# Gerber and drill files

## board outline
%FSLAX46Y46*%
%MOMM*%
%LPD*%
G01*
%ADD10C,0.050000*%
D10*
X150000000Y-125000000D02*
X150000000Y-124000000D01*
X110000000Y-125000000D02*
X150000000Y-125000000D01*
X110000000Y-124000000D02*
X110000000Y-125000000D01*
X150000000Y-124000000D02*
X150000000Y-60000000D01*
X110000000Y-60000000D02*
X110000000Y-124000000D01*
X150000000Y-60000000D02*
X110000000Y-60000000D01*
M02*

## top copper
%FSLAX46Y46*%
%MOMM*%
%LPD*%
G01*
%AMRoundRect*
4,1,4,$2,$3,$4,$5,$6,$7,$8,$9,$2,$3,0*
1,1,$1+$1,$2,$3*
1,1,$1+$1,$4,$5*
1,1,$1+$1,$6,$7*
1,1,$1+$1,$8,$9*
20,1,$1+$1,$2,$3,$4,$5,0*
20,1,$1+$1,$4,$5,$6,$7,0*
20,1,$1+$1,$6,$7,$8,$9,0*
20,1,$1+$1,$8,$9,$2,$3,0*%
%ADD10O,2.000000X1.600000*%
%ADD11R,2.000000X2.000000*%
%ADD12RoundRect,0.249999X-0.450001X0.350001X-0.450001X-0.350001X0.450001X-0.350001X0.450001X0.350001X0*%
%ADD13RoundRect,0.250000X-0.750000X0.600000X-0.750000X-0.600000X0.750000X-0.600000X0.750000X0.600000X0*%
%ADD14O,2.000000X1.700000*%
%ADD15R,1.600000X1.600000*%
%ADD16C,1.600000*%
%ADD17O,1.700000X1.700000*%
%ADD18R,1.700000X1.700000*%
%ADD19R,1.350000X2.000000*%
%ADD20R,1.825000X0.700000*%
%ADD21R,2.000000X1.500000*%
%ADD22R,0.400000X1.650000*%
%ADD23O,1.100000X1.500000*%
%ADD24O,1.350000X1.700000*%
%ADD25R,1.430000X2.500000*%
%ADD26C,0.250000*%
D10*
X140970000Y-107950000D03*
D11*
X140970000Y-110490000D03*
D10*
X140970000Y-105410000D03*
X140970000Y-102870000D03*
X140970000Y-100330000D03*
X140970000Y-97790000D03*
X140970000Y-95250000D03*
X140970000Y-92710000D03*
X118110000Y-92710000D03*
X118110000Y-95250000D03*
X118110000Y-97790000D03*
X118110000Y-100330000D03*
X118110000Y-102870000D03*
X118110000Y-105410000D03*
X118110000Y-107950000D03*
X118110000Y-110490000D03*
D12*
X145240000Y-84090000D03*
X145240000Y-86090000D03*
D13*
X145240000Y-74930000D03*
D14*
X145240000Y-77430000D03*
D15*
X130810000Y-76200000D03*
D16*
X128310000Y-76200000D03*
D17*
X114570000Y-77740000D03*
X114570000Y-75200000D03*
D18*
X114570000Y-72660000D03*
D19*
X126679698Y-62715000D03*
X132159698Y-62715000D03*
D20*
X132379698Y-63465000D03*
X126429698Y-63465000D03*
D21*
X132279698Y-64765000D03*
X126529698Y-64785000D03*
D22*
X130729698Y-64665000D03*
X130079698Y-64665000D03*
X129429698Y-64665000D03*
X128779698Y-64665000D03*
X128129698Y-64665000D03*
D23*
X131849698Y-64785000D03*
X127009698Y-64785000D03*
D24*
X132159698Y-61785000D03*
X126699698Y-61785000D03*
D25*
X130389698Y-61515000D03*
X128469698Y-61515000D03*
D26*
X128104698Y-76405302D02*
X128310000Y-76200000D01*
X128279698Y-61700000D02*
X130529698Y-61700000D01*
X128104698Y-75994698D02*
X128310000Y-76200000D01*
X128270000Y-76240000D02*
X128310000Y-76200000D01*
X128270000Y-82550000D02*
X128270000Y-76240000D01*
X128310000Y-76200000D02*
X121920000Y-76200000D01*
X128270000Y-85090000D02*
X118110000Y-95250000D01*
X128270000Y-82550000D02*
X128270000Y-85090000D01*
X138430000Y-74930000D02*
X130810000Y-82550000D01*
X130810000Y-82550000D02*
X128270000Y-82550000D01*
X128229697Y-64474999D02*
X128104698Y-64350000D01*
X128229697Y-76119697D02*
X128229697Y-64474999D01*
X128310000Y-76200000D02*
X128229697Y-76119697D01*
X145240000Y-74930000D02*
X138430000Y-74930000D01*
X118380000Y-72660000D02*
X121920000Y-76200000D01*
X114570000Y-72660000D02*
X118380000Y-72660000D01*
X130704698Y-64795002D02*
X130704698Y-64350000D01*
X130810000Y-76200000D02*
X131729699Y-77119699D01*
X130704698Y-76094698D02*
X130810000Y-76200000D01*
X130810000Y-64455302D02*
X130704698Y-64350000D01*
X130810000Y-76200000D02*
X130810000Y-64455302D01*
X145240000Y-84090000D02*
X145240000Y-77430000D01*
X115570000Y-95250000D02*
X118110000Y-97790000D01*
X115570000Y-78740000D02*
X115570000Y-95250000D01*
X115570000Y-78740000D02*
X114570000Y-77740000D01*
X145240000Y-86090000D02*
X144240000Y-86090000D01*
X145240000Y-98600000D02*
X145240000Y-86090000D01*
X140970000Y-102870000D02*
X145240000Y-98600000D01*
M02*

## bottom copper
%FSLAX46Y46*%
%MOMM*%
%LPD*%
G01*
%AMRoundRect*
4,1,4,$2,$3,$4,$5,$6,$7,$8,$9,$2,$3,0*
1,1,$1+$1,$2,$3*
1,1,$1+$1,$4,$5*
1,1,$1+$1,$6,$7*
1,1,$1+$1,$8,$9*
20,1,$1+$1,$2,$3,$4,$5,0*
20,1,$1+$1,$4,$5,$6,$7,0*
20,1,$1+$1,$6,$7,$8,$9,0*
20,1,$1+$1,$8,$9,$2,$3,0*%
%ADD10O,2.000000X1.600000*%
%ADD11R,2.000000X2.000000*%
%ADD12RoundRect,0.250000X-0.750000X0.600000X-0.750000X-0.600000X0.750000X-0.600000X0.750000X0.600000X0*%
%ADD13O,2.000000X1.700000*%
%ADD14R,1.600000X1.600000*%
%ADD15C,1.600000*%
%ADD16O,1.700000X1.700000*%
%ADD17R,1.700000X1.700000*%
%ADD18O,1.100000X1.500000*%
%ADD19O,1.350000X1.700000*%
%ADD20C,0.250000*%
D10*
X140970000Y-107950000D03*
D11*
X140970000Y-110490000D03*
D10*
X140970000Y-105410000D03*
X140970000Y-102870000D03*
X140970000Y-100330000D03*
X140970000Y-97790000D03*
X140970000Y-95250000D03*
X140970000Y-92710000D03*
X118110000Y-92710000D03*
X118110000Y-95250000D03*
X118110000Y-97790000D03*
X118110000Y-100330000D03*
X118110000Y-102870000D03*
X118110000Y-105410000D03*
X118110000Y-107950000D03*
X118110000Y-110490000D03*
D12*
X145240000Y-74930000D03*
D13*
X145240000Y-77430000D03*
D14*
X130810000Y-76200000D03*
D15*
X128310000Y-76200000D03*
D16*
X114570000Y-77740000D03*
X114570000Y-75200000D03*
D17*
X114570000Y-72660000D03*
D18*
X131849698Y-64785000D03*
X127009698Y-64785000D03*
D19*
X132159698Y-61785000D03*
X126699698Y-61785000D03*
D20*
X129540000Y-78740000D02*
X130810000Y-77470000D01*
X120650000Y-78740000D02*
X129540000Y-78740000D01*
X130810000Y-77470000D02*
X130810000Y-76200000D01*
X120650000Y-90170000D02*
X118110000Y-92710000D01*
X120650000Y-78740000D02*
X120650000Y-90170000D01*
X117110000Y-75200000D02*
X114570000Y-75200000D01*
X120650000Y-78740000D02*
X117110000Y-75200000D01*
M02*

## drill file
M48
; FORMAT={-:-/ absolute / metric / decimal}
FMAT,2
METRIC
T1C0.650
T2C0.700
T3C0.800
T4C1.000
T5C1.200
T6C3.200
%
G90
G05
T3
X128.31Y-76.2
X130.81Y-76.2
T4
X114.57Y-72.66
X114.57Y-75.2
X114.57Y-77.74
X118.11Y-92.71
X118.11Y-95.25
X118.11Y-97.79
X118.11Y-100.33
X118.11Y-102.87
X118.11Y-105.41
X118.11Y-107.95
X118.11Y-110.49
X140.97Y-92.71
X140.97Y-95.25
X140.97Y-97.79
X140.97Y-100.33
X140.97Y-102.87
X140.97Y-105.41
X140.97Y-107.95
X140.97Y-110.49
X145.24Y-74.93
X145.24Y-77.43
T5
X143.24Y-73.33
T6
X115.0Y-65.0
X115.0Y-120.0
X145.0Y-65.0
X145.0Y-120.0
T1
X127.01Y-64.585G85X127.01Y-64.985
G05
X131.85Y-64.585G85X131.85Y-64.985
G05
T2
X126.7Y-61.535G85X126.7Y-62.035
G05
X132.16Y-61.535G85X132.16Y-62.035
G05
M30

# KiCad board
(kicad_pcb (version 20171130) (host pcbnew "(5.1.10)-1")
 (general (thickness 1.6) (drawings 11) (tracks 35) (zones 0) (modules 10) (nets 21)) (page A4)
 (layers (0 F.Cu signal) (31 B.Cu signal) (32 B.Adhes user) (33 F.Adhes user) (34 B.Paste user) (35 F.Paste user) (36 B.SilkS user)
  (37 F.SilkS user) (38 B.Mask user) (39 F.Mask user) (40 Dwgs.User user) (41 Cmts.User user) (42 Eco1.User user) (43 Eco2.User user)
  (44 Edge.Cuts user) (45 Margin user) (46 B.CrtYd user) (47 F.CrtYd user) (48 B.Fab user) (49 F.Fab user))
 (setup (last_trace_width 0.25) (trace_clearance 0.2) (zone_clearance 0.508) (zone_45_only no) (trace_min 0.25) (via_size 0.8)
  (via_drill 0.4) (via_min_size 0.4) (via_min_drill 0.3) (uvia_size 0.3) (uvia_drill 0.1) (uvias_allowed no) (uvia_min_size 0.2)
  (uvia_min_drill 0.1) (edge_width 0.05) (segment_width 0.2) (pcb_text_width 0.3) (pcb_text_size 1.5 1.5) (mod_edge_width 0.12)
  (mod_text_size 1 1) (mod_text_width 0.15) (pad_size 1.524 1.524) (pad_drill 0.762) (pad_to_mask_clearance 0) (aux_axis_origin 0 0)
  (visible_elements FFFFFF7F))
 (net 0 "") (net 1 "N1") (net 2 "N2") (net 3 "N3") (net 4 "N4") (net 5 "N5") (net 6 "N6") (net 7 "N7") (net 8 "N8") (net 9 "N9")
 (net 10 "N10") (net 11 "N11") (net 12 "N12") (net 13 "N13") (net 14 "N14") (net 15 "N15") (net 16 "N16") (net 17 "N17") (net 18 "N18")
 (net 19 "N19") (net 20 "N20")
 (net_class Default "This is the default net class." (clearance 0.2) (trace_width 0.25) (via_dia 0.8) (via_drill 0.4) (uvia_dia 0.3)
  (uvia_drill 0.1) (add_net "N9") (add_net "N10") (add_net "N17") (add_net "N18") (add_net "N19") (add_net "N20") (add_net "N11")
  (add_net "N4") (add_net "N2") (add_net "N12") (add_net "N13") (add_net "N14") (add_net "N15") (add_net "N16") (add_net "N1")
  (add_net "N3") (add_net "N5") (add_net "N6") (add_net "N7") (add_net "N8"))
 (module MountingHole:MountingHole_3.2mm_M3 (layer F.Cu) (at 115 120)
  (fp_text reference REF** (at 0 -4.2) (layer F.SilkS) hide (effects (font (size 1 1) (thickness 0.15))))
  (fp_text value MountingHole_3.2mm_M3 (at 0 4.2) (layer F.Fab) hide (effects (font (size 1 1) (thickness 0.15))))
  (pad 1 np_thru_hole circle (at 0 0) (size 3.2 3.2) (drill 3.2) (layers *.Cu *.Mask)))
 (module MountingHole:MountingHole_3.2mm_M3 (layer F.Cu) (at 145 120)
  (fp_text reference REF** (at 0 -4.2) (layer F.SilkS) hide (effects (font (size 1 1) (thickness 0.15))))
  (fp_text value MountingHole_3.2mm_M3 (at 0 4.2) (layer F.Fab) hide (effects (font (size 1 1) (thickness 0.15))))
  (pad 1 np_thru_hole circle (at 0 0) (size 3.2 3.2) (drill 3.2) (layers *.Cu *.Mask)))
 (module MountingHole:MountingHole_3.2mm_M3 (layer F.Cu) (at 115 65)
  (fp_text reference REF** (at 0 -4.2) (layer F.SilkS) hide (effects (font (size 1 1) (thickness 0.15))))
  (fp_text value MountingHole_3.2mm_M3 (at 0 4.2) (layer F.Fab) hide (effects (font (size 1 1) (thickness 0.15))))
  (pad 1 np_thru_hole circle (at 0 0) (size 3.2 3.2) (drill 3.2) (layers *.Cu *.Mask)))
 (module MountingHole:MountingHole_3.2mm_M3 (layer F.Cu) (at 145 65)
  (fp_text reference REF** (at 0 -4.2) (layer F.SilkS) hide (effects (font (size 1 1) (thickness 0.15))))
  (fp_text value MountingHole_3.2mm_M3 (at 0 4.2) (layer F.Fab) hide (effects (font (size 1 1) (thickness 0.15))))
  (pad 1 np_thru_hole circle (at 0 0) (size 3.2 3.2) (drill 3.2) (layers *.Cu *.Mask)))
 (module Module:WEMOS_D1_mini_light (layer F.Cu) (at 140.97 110.49 180)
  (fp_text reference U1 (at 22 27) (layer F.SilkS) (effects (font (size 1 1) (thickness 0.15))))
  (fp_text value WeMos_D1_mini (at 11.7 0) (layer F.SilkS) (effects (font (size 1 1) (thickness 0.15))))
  (pad 2 thru_hole oval (at 0 2.54 180) (size 2 1.6) (drill 1) (layers *.Cu *.Mask) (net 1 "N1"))
  (pad 1 thru_hole rect (at 0 0 180) (size 2 2) (drill 1) (layers *.Cu *.Mask) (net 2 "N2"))
  (pad 3 thru_hole oval (at 0 5.08 180) (size 2 1.6) (drill 1) (layers *.Cu *.Mask) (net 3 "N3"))
  (pad 4 thru_hole oval (at 0 7.62 180) (size 2 1.6) (drill 1) (layers *.Cu *.Mask) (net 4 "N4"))
  (pad 5 thru_hole oval (at 0 10.16 180) (size 2 1.6) (drill 1) (layers *.Cu *.Mask) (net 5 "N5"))
  (pad 6 thru_hole oval (at 0 12.7 180) (size 2 1.6) (drill 1) (layers *.Cu *.Mask) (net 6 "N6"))
  (pad 7 thru_hole oval (at 0 15.24 180) (size 2 1.6) (drill 1) (layers *.Cu *.Mask) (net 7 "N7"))
  (pad 8 thru_hole oval (at 0 17.78 180) (size 2 1.6) (drill 1) (layers *.Cu *.Mask) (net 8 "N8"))
  (pad 9 thru_hole oval (at 22.86 17.78 180) (size 2 1.6) (drill 1) (layers *.Cu *.Mask) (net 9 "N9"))
  (pad 10 thru_hole oval (at 22.86 15.24 180) (size 2 1.6) (drill 1) (layers *.Cu *.Mask) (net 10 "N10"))
  (pad 11 thru_hole oval (at 22.86 12.7 180) (size 2 1.6) (drill 1) (layers *.Cu *.Mask) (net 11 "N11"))
  (pad 12 thru_hole oval (at 22.86 10.16 180) (size 2 1.6) (drill 1) (layers *.Cu *.Mask) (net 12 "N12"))
  (pad 13 thru_hole oval (at 22.86 7.62 180) (size 2 1.6) (drill 1) (layers *.Cu *.Mask) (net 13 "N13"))
  (pad 14 thru_hole oval (at 22.86 5.08 180) (size 2 1.6) (drill 1) (layers *.Cu *.Mask) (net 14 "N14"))
  (pad 15 thru_hole oval (at 22.86 2.54 180) (size 2 1.6) (drill 1) (layers *.Cu *.Mask) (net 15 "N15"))
  (pad 16 thru_hole oval (at 22.86 0 180) (size 2 1.6) (drill 1) (layers *.Cu *.Mask) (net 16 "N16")))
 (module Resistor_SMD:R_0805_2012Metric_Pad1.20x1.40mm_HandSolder (layer F.Cu) (at 145.24 85.09 270)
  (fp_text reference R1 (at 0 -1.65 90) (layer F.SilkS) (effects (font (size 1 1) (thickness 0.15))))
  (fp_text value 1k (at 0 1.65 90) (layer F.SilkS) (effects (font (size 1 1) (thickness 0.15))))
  (pad 1 smd roundrect (at -1 0 270) (size 1.2 1.4) (layers F.Cu F.Paste F.Mask) (roundrect_rratio 0.2083325) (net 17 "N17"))
  (pad 2 smd roundrect (at 1 0 270) (size 1.2 1.4) (layers F.Cu F.Paste F.Mask) (roundrect_rratio 0.2083325) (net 4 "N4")))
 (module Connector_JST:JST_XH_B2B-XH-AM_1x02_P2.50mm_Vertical (layer F.Cu) (at 145.24 74.93 270)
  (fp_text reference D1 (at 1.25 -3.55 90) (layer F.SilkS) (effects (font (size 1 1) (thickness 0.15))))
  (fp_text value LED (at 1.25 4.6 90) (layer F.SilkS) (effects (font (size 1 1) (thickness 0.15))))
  (pad 1 thru_hole roundrect (at 0 0 270) (size 1.7 2) (drill 1) (layers *.Cu *.Mask) (roundrect_rratio 0.1470588235294118) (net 10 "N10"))
  (pad 2 thru_hole oval (at 2.5 0 270) (size 1.7 2) (drill 1) (layers *.Cu *.Mask) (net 17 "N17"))
  (pad "" np_thru_hole circle (at -1.6 2 270) (size 1.2 1.2) (drill 1.2) (layers *.Cu *.Mask)))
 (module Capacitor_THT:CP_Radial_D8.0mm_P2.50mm (layer F.Cu) (at 130.81 76.2 180)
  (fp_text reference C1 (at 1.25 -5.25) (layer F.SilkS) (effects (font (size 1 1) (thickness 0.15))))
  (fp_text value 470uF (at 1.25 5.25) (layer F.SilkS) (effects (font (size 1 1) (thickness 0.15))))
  (pad 1 thru_hole rect (at 0 0 180) (size 1.6 1.6) (drill 0.8) (layers *.Cu *.Mask) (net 9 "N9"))
  (pad 2 thru_hole circle (at 2.5 0 180) (size 1.6 1.6) (drill 0.8) (layers *.Cu *.Mask) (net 10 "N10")))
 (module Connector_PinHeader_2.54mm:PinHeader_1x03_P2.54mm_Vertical (layer F.Cu) (at 114.57 72.66)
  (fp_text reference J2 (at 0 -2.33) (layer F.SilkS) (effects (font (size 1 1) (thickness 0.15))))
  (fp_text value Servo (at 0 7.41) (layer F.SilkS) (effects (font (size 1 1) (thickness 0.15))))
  (pad 3 thru_hole oval (at 0 5.08) (size 1.7 1.7) (drill 1) (layers *.Cu *.Mask) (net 11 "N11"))
  (pad 2 thru_hole oval (at 0 2.54) (size 1.7 1.7) (drill 1) (layers *.Cu *.Mask) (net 9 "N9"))
  (pad 1 thru_hole rect (at 0 0) (size 1.7 1.7) (drill 1) (layers *.Cu *.Mask) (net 10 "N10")))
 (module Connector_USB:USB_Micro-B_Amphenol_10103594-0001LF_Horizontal (layer F.Cu) (at 129.404698 62.9 180)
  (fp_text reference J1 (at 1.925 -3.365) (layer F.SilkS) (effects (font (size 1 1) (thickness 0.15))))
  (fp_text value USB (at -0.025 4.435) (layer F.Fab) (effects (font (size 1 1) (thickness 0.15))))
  (pad 6 smd rect (at 2.725 0.185 180) (size 1.35 2) (layers F.Cu F.Paste F.Mask) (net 10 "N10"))
  (pad 6 smd rect (at -2.755 0.185 180) (size 1.35 2) (layers F.Cu F.Paste F.Mask) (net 10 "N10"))
  (pad 6 smd rect (at -2.975 -0.565 180) (size 1.825 0.7) (layers F.Cu F.Paste F.Mask) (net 10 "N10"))
  (pad 6 smd rect (at 2.975 -0.565 180) (size 1.825 0.7) (layers F.Cu F.Paste F.Mask) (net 10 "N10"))
  (pad 6 smd rect (at -2.875 -1.865 180) (size 2 1.5) (layers F.Cu F.Paste F.Mask) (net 10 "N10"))
  (pad 6 smd rect (at 2.875 -1.885 180) (size 2 1.5) (layers F.Cu F.Paste F.Mask) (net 10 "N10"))
  (pad 1 smd rect (at -1.325 -1.765 270) (size 1.65 0.4) (layers F.Cu F.Paste F.Mask) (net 9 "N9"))
  (pad 2 smd rect (at -0.675 -1.765 270) (size 1.65 0.4) (layers F.Cu F.Paste F.Mask) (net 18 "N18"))
  (pad 3 smd rect (at -0.025 -1.765 270) (size 1.65 0.4) (layers F.Cu F.Paste F.Mask) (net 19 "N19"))
  (pad 4 smd rect (at 0.625 -1.765 270) (size 1.65 0.4) (layers F.Cu F.Paste F.Mask) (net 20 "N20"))
  (pad 5 smd rect (at 1.275 -1.765 270) (size 1.65 0.4) (layers F.Cu F.Paste F.Mask) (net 10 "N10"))
  (pad 6 thru_hole oval (at -2.445 -1.885 270) (size 1.5 1.1) (drill oval 1.05 0.65) (layers *.Cu *.Mask) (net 10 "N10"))
  (pad 6 thru_hole oval (at 2.395 -1.885 270) (size 1.5 1.1) (drill oval 1.05 0.65) (layers *.Cu *.Mask) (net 10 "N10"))
  (pad 6 thru_hole oval (at -2.755 1.115 270) (size 1.7 1.35) (drill oval 1.2 0.7) (layers *.Cu *.Mask) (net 10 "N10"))
  (pad 6 thru_hole oval (at 2.705 1.115 270) (size 1.7 1.35) (drill oval 1.2 0.7) (layers *.Cu *.Mask) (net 10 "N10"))
  (pad 6 smd rect (at -0.985 1.385 270) (size 2.5 1.43) (layers F.Cu F.Paste F.Mask) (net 10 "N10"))
  (pad 6 smd rect (at 0.935 1.385 270) (size 2.5 1.43) (layers F.Cu F.Paste F.Mask) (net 10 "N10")))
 (gr_line (start 150 125) (end 150 124) (layer Edge.Cuts) (width 0.05))
 (gr_line (start 110 125) (end 150 125) (layer Edge.Cuts) (width 0.05))
 (gr_line (start 110 124) (end 110 125) (layer Edge.Cuts) (width 0.05))
 (gr_line (start 150 124) (end 150 60) (layer Edge.Cuts) (width 0.05))
 (gr_line (start 110 60) (end 110 124) (layer Edge.Cuts) (width 0.05))
 (gr_line (start 150 60) (end 110 60) (layer Edge.Cuts) (width 0.05))
 (segment (start 128.104698 76.405302) (end 128.31 76.2) (width 0.25) (layer F.Cu) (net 10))
 (segment (start 128.279698 61.7) (end 130.529698 61.7) (width 0.25) (layer F.Cu) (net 10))
 (segment (start 128.104698 75.994698) (end 128.31 76.2) (width 0.25) (layer F.Cu) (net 10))
 (segment (start 128.27 76.24) (end 128.31 76.2) (width 0.25) (layer F.Cu) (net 10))
 (segment (start 128.27 82.55) (end 128.27 76.24) (width 0.25) (layer F.Cu) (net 10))
 (segment (start 128.31 76.2) (end 121.92 76.2) (width 0.25) (layer F.Cu) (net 10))
 (segment (start 128.27 85.09) (end 118.11 95.25) (width 0.25) (layer F.Cu) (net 10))
 (segment (start 128.27 82.55) (end 128.27 85.09) (width 0.25) (layer F.Cu) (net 10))
 (segment (start 138.43 74.93) (end 130.81 82.55) (width 0.25) (layer F.Cu) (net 10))
 (segment (start 130.81 82.55) (end 128.27 82.55) (width 0.25) (layer F.Cu) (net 10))
 (segment (start 128.229697 64.474999) (end 128.104698 64.35) (width 0.25) (layer F.Cu) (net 10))
 (segment (start 128.229697 76.119697) (end 128.229697 64.474999) (width 0.25) (layer F.Cu) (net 10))
 (segment (start 128.31 76.2) (end 128.229697 76.119697) (width 0.25) (layer F.Cu) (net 10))
 (segment (start 145.24 74.93) (end 138.43 74.93) (width 0.25) (layer F.Cu) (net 10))
 (segment (start 118.38 72.66) (end 121.92 76.2) (width 0.25) (layer F.Cu) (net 10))
 (segment (start 114.57 72.66) (end 118.38 72.66) (width 0.25) (layer F.Cu) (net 10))
 (segment (start 130.704698 64.795002) (end 130.704698 64.35) (width 0.25) (layer F.Cu) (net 9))
 (segment (start 130.81 76.2) (end 131.729699 77.119699) (width 0.25) (layer F.Cu) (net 9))
 (segment (start 130.704698 76.094698) (end 130.81 76.2) (width 0.25) (layer F.Cu) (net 9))
 (segment (start 129.54 78.74) (end 130.81 77.47) (width 0.25) (layer B.Cu) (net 9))
 (segment (start 120.65 78.74) (end 129.54 78.74) (width 0.25) (layer B.Cu) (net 9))
 (segment (start 130.81 77.47) (end 130.81 76.2) (width 0.25) (layer B.Cu) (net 9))
 (segment (start 120.65 90.17) (end 118.11 92.71) (width 0.25) (layer B.Cu) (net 9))
 (segment (start 120.65 78.74) (end 120.65 90.17) (width 0.25) (layer B.Cu) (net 9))
 (segment (start 130.81 64.455302) (end 130.704698 64.35) (width 0.25) (layer F.Cu) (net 9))
 (segment (start 130.81 76.2) (end 130.81 64.455302) (width 0.25) (layer F.Cu) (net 9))
 (segment (start 117.11 75.2) (end 114.57 75.2) (width 0.25) (layer B.Cu) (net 9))
 (segment (start 120.65 78.74) (end 117.11 75.2) (width 0.25) (layer B.Cu) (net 9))
 (segment (start 145.24 84.09) (end 145.24 77.43) (width 0.25) (layer F.Cu) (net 17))
 (segment (start 115.57 95.25) (end 118.11 97.79) (width 0.25) (layer F.Cu) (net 11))
 (segment (start 115.57 78.74) (end 115.57 95.25) (width 0.25) (layer F.Cu) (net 11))
 (segment (start 115.57 78.74) (end 114.57 77.74) (width 0.25) (layer F.Cu) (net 11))
 (segment (start 145.24 86.09) (end 144.24 86.09) (width 0.25) (layer F.Cu) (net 4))
 (segment (start 145.24 98.6) (end 145.24 86.09) (width 0.25) (layer F.Cu) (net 4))
 (segment (start 140.97 102.87) (end 145.24 98.6) (width 0.25) (layer F.Cu) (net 4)))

